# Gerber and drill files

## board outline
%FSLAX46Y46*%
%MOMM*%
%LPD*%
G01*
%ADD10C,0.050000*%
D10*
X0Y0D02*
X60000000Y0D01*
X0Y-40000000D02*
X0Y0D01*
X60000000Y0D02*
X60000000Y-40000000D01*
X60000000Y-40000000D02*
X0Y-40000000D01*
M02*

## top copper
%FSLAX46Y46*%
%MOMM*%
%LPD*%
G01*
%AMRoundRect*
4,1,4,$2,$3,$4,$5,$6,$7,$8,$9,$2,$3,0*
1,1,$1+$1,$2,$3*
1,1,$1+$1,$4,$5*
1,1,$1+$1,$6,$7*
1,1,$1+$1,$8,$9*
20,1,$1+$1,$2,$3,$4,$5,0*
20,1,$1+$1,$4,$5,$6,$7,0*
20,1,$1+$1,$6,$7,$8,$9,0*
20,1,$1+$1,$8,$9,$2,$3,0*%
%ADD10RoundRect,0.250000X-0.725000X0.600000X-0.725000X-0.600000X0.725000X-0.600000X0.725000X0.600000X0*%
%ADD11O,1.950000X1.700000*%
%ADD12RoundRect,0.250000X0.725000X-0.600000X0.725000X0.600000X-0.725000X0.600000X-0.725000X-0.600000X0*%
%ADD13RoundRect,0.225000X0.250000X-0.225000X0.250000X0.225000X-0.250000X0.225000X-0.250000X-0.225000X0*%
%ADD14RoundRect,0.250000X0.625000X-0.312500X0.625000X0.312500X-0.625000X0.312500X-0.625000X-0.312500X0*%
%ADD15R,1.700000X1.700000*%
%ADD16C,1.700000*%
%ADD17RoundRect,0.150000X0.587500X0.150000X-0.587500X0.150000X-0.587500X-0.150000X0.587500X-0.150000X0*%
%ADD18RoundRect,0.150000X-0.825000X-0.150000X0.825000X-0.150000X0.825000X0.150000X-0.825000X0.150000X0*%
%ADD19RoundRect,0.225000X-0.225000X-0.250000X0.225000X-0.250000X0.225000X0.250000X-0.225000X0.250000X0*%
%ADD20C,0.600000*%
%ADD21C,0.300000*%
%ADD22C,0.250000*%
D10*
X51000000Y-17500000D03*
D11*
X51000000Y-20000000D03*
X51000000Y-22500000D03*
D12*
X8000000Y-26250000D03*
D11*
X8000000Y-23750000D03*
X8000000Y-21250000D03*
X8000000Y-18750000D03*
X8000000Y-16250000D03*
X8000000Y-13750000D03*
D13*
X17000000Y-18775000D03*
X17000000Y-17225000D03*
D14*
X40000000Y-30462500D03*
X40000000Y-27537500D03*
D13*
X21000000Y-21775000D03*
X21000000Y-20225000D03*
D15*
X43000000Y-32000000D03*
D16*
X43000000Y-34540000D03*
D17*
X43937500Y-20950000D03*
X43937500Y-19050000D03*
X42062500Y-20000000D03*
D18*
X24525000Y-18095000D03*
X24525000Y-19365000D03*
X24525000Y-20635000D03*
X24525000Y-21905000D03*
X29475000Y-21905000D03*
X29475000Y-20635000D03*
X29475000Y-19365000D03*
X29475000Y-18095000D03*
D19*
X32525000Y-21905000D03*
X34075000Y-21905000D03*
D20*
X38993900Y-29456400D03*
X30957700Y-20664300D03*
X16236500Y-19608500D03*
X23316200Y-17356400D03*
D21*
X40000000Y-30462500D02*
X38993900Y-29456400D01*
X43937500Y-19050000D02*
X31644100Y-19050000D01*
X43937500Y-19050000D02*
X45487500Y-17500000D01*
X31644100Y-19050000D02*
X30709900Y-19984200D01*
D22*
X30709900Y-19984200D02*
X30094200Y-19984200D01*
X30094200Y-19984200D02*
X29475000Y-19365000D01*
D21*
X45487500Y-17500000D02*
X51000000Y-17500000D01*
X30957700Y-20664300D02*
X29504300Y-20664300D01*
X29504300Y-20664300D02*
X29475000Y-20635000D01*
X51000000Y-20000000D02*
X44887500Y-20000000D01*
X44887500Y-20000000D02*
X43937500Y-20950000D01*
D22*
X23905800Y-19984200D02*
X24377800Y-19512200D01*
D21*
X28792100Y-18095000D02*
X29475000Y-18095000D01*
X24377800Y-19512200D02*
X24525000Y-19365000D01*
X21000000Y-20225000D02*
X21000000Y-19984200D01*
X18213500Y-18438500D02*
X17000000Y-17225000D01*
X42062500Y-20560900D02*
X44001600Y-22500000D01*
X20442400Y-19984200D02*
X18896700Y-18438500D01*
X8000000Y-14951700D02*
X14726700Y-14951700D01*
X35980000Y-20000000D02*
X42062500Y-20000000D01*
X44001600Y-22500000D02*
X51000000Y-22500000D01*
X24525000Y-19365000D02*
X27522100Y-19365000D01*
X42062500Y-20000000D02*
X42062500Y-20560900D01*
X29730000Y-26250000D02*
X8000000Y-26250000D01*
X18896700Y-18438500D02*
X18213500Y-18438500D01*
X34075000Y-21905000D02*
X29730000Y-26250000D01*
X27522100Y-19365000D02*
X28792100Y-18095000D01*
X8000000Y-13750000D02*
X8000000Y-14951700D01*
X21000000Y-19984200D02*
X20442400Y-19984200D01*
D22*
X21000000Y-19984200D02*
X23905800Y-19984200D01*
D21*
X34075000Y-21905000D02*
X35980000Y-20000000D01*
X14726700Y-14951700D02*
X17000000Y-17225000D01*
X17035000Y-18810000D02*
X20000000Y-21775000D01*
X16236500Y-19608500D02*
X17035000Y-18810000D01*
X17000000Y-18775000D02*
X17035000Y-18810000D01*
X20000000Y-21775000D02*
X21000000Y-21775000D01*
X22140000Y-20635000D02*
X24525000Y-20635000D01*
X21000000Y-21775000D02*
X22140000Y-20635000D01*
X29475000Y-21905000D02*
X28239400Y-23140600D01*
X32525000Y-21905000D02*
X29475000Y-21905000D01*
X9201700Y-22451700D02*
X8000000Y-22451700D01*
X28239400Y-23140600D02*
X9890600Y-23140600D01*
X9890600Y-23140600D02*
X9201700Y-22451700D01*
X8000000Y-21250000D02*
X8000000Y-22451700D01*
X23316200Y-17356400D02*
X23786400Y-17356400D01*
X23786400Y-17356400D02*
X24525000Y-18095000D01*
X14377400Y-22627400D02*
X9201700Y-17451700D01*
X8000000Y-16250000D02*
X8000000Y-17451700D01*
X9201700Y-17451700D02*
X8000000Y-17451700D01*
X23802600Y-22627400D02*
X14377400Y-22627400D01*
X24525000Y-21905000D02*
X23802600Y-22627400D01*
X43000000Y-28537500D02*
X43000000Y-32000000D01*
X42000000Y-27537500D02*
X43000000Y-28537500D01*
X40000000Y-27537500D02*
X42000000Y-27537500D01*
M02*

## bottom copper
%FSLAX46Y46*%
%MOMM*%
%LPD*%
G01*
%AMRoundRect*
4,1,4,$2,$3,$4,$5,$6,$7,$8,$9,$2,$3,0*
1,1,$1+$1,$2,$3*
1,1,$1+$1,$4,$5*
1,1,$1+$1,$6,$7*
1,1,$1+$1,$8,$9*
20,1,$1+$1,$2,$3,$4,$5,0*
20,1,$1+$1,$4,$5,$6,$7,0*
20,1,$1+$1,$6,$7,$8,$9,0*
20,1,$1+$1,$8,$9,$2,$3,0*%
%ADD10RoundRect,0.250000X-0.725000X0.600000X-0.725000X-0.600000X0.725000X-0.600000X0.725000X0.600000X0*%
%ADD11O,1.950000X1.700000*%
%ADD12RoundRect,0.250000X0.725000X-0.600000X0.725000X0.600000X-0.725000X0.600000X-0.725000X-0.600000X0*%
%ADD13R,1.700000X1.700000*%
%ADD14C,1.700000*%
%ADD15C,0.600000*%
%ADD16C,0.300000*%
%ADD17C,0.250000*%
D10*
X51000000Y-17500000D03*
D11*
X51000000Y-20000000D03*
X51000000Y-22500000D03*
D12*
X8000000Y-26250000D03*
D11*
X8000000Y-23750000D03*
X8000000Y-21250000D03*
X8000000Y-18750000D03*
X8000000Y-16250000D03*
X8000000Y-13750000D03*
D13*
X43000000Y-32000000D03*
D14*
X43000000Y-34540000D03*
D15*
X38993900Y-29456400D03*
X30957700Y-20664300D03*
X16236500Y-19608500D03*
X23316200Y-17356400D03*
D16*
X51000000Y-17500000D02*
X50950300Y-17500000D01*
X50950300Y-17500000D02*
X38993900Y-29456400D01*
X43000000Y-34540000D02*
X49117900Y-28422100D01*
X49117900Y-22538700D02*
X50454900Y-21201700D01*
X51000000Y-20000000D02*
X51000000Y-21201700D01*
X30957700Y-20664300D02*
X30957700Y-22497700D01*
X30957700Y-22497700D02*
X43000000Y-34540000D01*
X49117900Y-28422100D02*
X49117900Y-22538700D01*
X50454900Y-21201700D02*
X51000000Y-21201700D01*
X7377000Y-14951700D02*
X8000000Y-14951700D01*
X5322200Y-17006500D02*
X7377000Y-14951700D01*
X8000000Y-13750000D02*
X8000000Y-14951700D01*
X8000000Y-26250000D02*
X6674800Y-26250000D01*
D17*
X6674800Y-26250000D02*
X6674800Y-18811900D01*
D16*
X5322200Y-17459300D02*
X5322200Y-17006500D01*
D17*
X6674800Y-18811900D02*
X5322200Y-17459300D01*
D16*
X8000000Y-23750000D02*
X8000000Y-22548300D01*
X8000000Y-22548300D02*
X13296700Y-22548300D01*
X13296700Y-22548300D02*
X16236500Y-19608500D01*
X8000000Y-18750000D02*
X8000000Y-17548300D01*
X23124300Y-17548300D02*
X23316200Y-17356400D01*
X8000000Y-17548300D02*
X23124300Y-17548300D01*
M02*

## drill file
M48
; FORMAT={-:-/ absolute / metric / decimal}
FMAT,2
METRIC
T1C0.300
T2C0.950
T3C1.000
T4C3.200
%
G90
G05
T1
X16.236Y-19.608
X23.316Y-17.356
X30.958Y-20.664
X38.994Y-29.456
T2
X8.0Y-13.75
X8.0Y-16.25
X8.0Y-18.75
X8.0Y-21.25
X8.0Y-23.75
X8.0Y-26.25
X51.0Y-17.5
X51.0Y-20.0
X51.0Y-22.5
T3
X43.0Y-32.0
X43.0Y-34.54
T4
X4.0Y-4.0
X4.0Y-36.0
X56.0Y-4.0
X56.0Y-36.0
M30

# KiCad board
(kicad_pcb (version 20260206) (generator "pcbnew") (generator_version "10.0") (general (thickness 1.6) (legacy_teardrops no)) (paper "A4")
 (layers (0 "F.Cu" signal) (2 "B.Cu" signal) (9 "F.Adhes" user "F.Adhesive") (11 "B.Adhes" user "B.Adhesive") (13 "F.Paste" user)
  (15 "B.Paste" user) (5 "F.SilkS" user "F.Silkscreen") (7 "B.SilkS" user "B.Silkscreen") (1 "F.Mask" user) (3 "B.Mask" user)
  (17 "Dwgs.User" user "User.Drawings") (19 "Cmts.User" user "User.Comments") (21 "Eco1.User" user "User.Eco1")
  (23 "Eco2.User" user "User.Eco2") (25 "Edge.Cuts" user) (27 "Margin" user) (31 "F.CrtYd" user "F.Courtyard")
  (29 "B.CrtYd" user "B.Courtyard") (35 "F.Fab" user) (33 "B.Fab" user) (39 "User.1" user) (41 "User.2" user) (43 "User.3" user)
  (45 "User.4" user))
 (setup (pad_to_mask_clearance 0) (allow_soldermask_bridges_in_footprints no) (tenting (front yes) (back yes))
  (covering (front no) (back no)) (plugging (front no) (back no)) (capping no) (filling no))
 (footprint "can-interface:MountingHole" (layer "F.Cu") (at 56 36)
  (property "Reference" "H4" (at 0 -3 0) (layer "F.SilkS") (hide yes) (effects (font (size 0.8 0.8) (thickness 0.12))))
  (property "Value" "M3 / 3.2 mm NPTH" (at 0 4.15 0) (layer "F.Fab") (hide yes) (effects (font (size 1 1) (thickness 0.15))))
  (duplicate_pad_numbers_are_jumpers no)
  (pad "" np_thru_hole circle (at 0 0) (size 3.2 3.2) (drill 3.2) (layers "*.Cu" "*.Mask")))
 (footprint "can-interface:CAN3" (layer "F.Cu") (at 51 17.5 -90)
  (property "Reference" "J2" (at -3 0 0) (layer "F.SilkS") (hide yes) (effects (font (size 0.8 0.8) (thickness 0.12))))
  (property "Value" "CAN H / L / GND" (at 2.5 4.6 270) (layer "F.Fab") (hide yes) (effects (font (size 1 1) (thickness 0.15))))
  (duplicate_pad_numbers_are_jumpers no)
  (pad "1" thru_hole roundrect (at 0 0 270) (size 1.7 1.95) (drill 0.95) (layers "*.Cu" "*.Mask") (remove_unused_layers no)
   (roundrect_rratio 0.147059) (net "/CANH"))
  (pad "2" thru_hole oval (at 2.5 0 270) (size 1.7 1.95) (drill 0.95) (layers "*.Cu" "*.Mask") (remove_unused_layers no) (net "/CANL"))
  (pad "3" thru_hole oval (at 5 0 270) (size 1.7 1.95) (drill 0.95) (layers "*.Cu" "*.Mask") (remove_unused_layers no) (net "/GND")))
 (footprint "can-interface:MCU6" (layer "F.Cu") (at 8 26.25 90)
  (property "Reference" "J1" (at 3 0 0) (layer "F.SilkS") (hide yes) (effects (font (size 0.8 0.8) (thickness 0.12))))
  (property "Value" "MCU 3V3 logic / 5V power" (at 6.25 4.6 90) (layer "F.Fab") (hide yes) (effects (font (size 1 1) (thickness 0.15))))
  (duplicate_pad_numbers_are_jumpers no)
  (pad "1" thru_hole roundrect (at 0 0 90) (size 1.7 1.95) (drill 0.95) (layers "*.Cu" "*.Mask") (remove_unused_layers no)
   (roundrect_rratio 0.147059) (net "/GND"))
  (pad "2" thru_hole oval (at 2.5 0 90) (size 1.7 1.95) (drill 0.95) (layers "*.Cu" "*.Mask") (remove_unused_layers no) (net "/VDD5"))
  (pad "3" thru_hole oval (at 5 0 90) (size 1.7 1.95) (drill 0.95) (layers "*.Cu" "*.Mask") (remove_unused_layers no) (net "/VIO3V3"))
  (pad "4" thru_hole oval (at 7.5 0 90) (size 1.7 1.95) (drill 0.95) (layers "*.Cu" "*.Mask") (remove_unused_layers no) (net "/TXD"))
  (pad "5" thru_hole oval (at 10 0 90) (size 1.7 1.95) (drill 0.95) (layers "*.Cu" "*.Mask") (remove_unused_layers no) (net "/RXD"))
  (pad "6" thru_hole oval (at 12.5 0 90) (size 1.7 1.95) (drill 0.95) (layers "*.Cu" "*.Mask") (remove_unused_layers no) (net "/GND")))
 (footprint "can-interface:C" (layer "F.Cu") (at 17 18 90)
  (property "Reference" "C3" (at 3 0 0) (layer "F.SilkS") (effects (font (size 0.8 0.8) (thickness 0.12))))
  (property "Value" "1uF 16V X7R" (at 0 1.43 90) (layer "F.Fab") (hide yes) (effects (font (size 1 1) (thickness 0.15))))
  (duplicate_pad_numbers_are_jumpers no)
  (pad "1" smd roundrect (at -0.775 0 90) (size 0.9 0.95) (layers "F.Cu" "F.Mask" "F.Paste") (roundrect_rratio 0.25) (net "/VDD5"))
  (pad "2" smd roundrect (at 0.775 0 90) (size 0.9 0.95) (layers "F.Cu" "F.Mask" "F.Paste") (roundrect_rratio 0.25) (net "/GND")))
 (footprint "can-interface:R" (layer "F.Cu") (at 40 29 90)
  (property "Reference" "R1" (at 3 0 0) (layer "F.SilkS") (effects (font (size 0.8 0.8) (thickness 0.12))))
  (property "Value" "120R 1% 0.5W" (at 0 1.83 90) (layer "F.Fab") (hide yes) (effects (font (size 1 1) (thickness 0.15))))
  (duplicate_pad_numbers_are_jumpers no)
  (pad "1" smd roundrect (at -1.4625 0 90) (size 1.125 1.75) (layers "F.Cu" "F.Mask" "F.Paste") (roundrect_rratio 0.222222) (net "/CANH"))
  (pad "2" smd roundrect (at 1.4625 0 90) (size 1.125 1.75) (layers "F.Cu" "F.Mask" "F.Paste") (roundrect_rratio 0.222222) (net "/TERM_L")))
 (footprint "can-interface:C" (layer "F.Cu") (at 21 21 90)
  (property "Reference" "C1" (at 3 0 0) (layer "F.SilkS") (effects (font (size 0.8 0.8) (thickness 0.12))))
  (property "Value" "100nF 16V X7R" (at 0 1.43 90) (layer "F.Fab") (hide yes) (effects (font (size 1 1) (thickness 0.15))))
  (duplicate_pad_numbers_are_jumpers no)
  (pad "1" smd roundrect (at -0.775 0 90) (size 0.9 0.95) (layers "F.Cu" "F.Mask" "F.Paste") (roundrect_rratio 0.25) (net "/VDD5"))
  (pad "2" smd roundrect (at 0.775 0 90) (size 0.9 0.95) (layers "F.Cu" "F.Mask" "F.Paste") (roundrect_rratio 0.25) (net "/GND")))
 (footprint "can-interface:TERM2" (layer "F.Cu") (at 43 32)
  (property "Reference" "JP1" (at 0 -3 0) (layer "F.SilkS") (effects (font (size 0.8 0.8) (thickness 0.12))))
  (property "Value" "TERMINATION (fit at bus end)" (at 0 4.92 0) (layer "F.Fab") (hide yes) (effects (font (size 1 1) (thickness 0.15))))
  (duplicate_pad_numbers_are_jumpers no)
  (pad "1" thru_hole rect (at 0 0) (size 1.7 1.7) (drill 1) (layers "*.Cu" "*.Mask") (remove_unused_layers no) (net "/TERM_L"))
  (pad "2" thru_hole circle (at 0 2.54) (size 1.7 1.7) (drill 1) (layers "*.Cu" "*.Mask") (remove_unused_layers no) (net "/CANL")))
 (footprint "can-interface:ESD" (layer "F.Cu") (at 43 20 180)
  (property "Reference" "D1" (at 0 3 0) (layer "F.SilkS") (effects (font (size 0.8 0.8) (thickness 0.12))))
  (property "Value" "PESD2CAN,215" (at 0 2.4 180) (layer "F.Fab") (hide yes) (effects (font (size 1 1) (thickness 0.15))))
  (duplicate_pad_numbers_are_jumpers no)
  (pad "1" smd roundrect (at -0.9375 -0.95 180) (size 1.475 0.6) (layers "F.Cu" "F.Mask" "F.Paste") (roundrect_rratio 0.25) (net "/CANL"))
  (pad "2" smd roundrect (at -0.9375 0.95 180) (size 1.475 0.6) (layers "F.Cu" "F.Mask" "F.Paste") (roundrect_rratio 0.25) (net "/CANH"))
  (pad "3" smd roundrect (at 0.9375 0 180) (size 1.475 0.6) (layers "F.Cu" "F.Mask" "F.Paste") (roundrect_rratio 0.25) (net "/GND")))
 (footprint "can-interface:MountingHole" (layer "F.Cu") (at 4 36)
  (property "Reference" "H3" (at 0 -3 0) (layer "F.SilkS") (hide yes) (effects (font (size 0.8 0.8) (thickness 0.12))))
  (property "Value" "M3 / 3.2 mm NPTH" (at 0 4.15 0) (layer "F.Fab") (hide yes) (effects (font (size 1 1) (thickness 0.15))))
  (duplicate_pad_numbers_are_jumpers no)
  (pad "" np_thru_hole circle (at 0 0) (size 3.2 3.2) (drill 3.2) (layers "*.Cu" "*.Mask")))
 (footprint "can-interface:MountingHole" (layer "F.Cu") (at 4 4)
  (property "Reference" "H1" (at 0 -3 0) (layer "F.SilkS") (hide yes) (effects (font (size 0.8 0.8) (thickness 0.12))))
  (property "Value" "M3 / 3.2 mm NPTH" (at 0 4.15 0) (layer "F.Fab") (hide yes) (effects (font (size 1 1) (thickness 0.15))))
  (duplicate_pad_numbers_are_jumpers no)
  (pad "" np_thru_hole circle (at 0 0) (size 3.2 3.2) (drill 3.2) (layers "*.Cu" "*.Mask")))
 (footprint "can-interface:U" (layer "F.Cu") (at 27 20)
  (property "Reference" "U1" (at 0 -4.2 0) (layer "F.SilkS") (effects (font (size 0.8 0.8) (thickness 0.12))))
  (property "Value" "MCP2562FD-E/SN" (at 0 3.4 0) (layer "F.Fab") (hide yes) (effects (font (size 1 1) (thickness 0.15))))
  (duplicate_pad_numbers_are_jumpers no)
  (pad "1" smd roundrect (at -2.475 -1.905) (size 1.95 0.6) (layers "F.Cu" "F.Mask" "F.Paste") (roundrect_rratio 0.25) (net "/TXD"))
  (pad "2" smd roundrect (at -2.475 -0.635) (size 1.95 0.6) (layers "F.Cu" "F.Mask" "F.Paste") (roundrect_rratio 0.25) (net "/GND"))
  (pad "3" smd roundrect (at -2.475 0.635) (size 1.95 0.6) (layers "F.Cu" "F.Mask" "F.Paste") (roundrect_rratio 0.25) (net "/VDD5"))
  (pad "4" smd roundrect (at -2.475 1.905) (size 1.95 0.6) (layers "F.Cu" "F.Mask" "F.Paste") (roundrect_rratio 0.25) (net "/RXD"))
  (pad "5" smd roundrect (at 2.475 1.905) (size 1.95 0.6) (layers "F.Cu" "F.Mask" "F.Paste") (roundrect_rratio 0.25) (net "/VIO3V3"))
  (pad "6" smd roundrect (at 2.475 0.635) (size 1.95 0.6) (layers "F.Cu" "F.Mask" "F.Paste") (roundrect_rratio 0.25) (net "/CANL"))
  (pad "7" smd roundrect (at 2.475 -0.635) (size 1.95 0.6) (layers "F.Cu" "F.Mask" "F.Paste") (roundrect_rratio 0.25) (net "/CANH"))
  (pad "8" smd roundrect (at 2.475 -1.905) (size 1.95 0.6) (layers "F.Cu" "F.Mask" "F.Paste") (roundrect_rratio 0.25) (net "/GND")))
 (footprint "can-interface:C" (layer "F.Cu") (at 33.3 21.905)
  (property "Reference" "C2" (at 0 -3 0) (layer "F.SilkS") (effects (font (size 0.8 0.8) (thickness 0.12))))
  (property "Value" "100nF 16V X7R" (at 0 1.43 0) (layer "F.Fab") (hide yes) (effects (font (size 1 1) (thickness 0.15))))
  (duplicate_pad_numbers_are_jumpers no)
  (pad "1" smd roundrect (at -0.775 0) (size 0.9 0.95) (layers "F.Cu" "F.Mask" "F.Paste") (roundrect_rratio 0.25) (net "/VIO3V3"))
  (pad "2" smd roundrect (at 0.775 0) (size 0.9 0.95) (layers "F.Cu" "F.Mask" "F.Paste") (roundrect_rratio 0.25) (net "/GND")))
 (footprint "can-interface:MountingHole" (layer "F.Cu") (at 56 4)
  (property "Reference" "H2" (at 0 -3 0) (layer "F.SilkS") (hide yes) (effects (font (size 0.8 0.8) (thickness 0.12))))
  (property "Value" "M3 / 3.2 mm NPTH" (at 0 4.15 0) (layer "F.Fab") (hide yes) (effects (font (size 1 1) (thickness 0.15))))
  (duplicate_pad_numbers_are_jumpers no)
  (pad "" np_thru_hole circle (at 0 0) (size 3.2 3.2) (drill 3.2) (layers "*.Cu" "*.Mask")))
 (gr_line (start 0 0) (end 60 0) (stroke (width 0.05) (type default)) (layer "Edge.Cuts"))
 (gr_line (start 0 40) (end 0 0) (stroke (width 0.05) (type default)) (layer "Edge.Cuts"))
 (gr_line (start 60 0) (end 60 40) (stroke (width 0.05) (type default)) (layer "Edge.Cuts"))
 (gr_line (start 60 40) (end 0 40) (stroke (width 0.05) (type default)) (layer "Edge.Cuts"))
 (segment (start 40 30.4625) (end 38.9939 29.4564) (width 0.3) (layer "F.Cu") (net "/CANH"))
 (segment (start 43.9375 19.05) (end 31.6441 19.05) (width 0.3) (layer "F.Cu") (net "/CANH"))
 (segment (start 43.9375 19.05) (end 45.4875 17.5) (width 0.3) (layer "F.Cu") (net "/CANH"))
 (segment (start 31.6441 19.05) (end 30.7099 19.9842) (width 0.3) (layer "F.Cu") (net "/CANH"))
 (segment (start 30.7099 19.9842) (end 30.0942 19.9842) (width 0.25) (layer "F.Cu") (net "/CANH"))
 (segment (start 30.0942 19.9842) (end 29.475 19.365) (width 0.25) (layer "F.Cu") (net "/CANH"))
 (segment (start 45.4875 17.5) (end 51 17.5) (width 0.3) (layer "F.Cu") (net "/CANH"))
 (via (at 38.9939 29.4564) (size 0.6) (drill 0.3) (layers "F.Cu" "B.Cu") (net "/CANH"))
 (segment (start 51 17.5) (end 50.9503 17.5) (width 0.3) (layer "B.Cu") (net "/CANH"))
 (segment (start 50.9503 17.5) (end 38.9939 29.4564) (width 0.3) (layer "B.Cu") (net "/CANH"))
 (segment (start 30.9577 20.6643) (end 29.5043 20.6643) (width 0.3) (layer "F.Cu") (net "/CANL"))
 (segment (start 29.5043 20.6643) (end 29.475 20.635) (width 0.3) (layer "F.Cu") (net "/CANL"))
 (segment (start 51 20) (end 44.8875 20) (width 0.3) (layer "F.Cu") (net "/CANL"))
 (segment (start 44.8875 20) (end 43.9375 20.95) (width 0.3) (layer "F.Cu") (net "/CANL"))
 (via (at 30.9577 20.6643) (size 0.6) (drill 0.3) (layers "F.Cu" "B.Cu") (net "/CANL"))
 (segment (start 43 34.54) (end 49.1179 28.4221) (width 0.3) (layer "B.Cu") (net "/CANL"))
 (segment (start 49.1179 22.5387) (end 50.4549 21.2017) (width 0.3) (layer "B.Cu") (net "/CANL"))
 (segment (start 51 20) (end 51 21.2017) (width 0.3) (layer "B.Cu") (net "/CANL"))
 (segment (start 30.9577 20.6643) (end 30.9577 22.4977) (width 0.3) (layer "B.Cu") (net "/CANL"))
 (segment (start 30.9577 22.4977) (end 43 34.54) (width 0.3) (layer "B.Cu") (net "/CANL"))
 (segment (start 49.1179 28.4221) (end 49.1179 22.5387) (width 0.3) (layer "B.Cu") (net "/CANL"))
 (segment (start 50.4549 21.2017) (end 51 21.2017) (width 0.3) (layer "B.Cu") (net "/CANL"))
 (segment (start 23.9058 19.9842) (end 24.3778 19.5122) (width 0.25) (layer "F.Cu") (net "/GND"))
 (segment (start 28.7921 18.095) (end 29.475 18.095) (width 0.3) (layer "F.Cu") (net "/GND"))
 (segment (start 24.3778 19.5122) (end 24.525 19.365) (width 0.3) (layer "F.Cu") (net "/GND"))
 (segment (start 21 20.225) (end 21 19.9842) (width 0.3) (layer "F.Cu") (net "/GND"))
 (segment (start 18.2135 18.4385) (end 17 17.225) (width 0.3) (layer "F.Cu") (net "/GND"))
 (segment (start 42.0625 20.5609) (end 44.0016 22.5) (width 0.3) (layer "F.Cu") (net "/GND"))
 (segment (start 20.4424 19.9842) (end 18.8967 18.4385) (width 0.3) (layer "F.Cu") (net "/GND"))
 (segment (start 8 14.9517) (end 14.7267 14.9517) (width 0.3) (layer "F.Cu") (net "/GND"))
 (segment (start 35.98 20) (end 42.0625 20) (width 0.3) (layer "F.Cu") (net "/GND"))
 (segment (start 44.0016 22.5) (end 51 22.5) (width 0.3) (layer "F.Cu") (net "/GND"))
 (segment (start 24.525 19.365) (end 27.5221 19.365) (width 0.3) (layer "F.Cu") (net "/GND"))
 (segment (start 42.0625 20) (end 42.0625 20.5609) (width 0.3) (layer "F.Cu") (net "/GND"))
 (segment (start 29.73 26.25) (end 8 26.25) (width 0.3) (layer "F.Cu") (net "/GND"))
 (segment (start 18.8967 18.4385) (end 18.2135 18.4385) (width 0.3) (layer "F.Cu") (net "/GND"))
 (segment (start 34.075 21.905) (end 29.73 26.25) (width 0.3) (layer "F.Cu") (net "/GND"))
 (segment (start 27.5221 19.365) (end 28.7921 18.095) (width 0.3) (layer "F.Cu") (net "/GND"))
 (segment (start 8 13.75) (end 8 14.9517) (width 0.3) (layer "F.Cu") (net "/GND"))
 (segment (start 21 19.9842) (end 20.4424 19.9842) (width 0.3) (layer "F.Cu") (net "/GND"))
 (segment (start 21 19.9842) (end 23.9058 19.9842) (width 0.25) (layer "F.Cu") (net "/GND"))
 (segment (start 34.075 21.905) (end 35.98 20) (width 0.3) (layer "F.Cu") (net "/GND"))
 (segment (start 14.7267 14.9517) (end 17 17.225) (width 0.3) (layer "F.Cu") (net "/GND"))
 (segment (start 7.377 14.9517) (end 8 14.9517) (width 0.3) (layer "B.Cu") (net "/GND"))
 (segment (start 5.3222 17.0065) (end 7.377 14.9517) (width 0.3) (layer "B.Cu") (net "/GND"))
 (segment (start 8 13.75) (end 8 14.9517) (width 0.3) (layer "B.Cu") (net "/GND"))
 (segment (start 8 26.25) (end 6.6748 26.25) (width 0.3) (layer "B.Cu") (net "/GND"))
 (segment (start 6.6748 26.25) (end 6.6748 18.8119) (width 0.25) (layer "B.Cu") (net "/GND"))
 (segment (start 5.3222 17.4593) (end 5.3222 17.0065) (width 0.3) (layer "B.Cu") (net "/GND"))
 (segment (start 6.6748 18.8119) (end 5.3222 17.4593) (width 0.25) (layer "B.Cu") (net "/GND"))
 (segment (start 17.035 18.81) (end 20 21.775) (width 0.3) (layer "F.Cu") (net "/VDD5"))
 (segment (start 16.2365 19.6085) (end 17.035 18.81) (width 0.3) (layer "F.Cu") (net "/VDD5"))
 (segment (start 17 18.775) (end 17.035 18.81) (width 0.3) (layer "F.Cu") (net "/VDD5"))
 (segment (start 20 21.775) (end 21 21.775) (width 0.3) (layer "F.Cu") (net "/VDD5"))
 (segment (start 22.14 20.635) (end 24.525 20.635) (width 0.3) (layer "F.Cu") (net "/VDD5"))
 (segment (start 21 21.775) (end 22.14 20.635) (width 0.3) (layer "F.Cu") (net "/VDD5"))
 (via (at 16.2365 19.6085) (size 0.6) (drill 0.3) (layers "F.Cu" "B.Cu") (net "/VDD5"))
 (segment (start 8 23.75) (end 8 22.5483) (width 0.3) (layer "B.Cu") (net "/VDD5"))
 (segment (start 8 22.5483) (end 13.2967 22.5483) (width 0.3) (layer "B.Cu") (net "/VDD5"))
 (segment (start 13.2967 22.5483) (end 16.2365 19.6085) (width 0.3) (layer "B.Cu") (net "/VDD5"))
 (segment (start 29.475 21.905) (end 28.2394 23.1406) (width 0.3) (layer "F.Cu") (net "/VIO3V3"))
 (segment (start 32.525 21.905) (end 29.475 21.905) (width 0.3) (layer "F.Cu") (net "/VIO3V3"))
 (segment (start 9.2017 22.4517) (end 8 22.4517) (width 0.3) (layer "F.Cu") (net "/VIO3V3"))
 (segment (start 28.2394 23.1406) (end 9.8906 23.1406) (width 0.3) (layer "F.Cu") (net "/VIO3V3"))
 (segment (start 9.8906 23.1406) (end 9.2017 22.4517) (width 0.3) (layer "F.Cu") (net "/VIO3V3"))
 (segment (start 8 21.25) (end 8 22.4517) (width 0.3) (layer "F.Cu") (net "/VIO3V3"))
 (segment (start 23.3162 17.3564) (end 23.7864 17.3564) (width 0.3) (layer "F.Cu") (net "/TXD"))
 (segment (start 23.7864 17.3564) (end 24.525 18.095) (width 0.3) (layer "F.Cu") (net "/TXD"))
 (via (at 23.3162 17.3564) (size 0.6) (drill 0.3) (layers "F.Cu" "B.Cu") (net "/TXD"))
 (segment (start 8 18.75) (end 8 17.5483) (width 0.3) (layer "B.Cu") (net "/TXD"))
 (segment (start 23.1243 17.5483) (end 23.3162 17.3564) (width 0.3) (layer "B.Cu") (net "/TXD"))
 (segment (start 8 17.5483) (end 23.1243 17.5483) (width 0.3) (layer "B.Cu") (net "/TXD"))
 (segment (start 14.3774 22.6274) (end 9.2017 17.4517) (width 0.3) (layer "F.Cu") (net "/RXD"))
 (segment (start 8 16.25) (end 8 17.4517) (width 0.3) (layer "F.Cu") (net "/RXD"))
 (segment (start 9.2017 17.4517) (end 8 17.4517) (width 0.3) (layer "F.Cu") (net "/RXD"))
 (segment (start 23.8026 22.6274) (end 14.3774 22.6274) (width 0.3) (layer "F.Cu") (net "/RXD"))
 (segment (start 24.525 21.905) (end 23.8026 22.6274) (width 0.3) (layer "F.Cu") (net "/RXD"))
 (segment (start 43 28.5375) (end 43 32) (width 0.3) (layer "F.Cu") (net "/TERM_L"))
 (segment (start 42 27.5375) (end 43 28.5375) (width 0.3) (layer "F.Cu") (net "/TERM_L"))
 (segment (start 40 27.5375) (end 42 27.5375) (width 0.3) (layer "F.Cu") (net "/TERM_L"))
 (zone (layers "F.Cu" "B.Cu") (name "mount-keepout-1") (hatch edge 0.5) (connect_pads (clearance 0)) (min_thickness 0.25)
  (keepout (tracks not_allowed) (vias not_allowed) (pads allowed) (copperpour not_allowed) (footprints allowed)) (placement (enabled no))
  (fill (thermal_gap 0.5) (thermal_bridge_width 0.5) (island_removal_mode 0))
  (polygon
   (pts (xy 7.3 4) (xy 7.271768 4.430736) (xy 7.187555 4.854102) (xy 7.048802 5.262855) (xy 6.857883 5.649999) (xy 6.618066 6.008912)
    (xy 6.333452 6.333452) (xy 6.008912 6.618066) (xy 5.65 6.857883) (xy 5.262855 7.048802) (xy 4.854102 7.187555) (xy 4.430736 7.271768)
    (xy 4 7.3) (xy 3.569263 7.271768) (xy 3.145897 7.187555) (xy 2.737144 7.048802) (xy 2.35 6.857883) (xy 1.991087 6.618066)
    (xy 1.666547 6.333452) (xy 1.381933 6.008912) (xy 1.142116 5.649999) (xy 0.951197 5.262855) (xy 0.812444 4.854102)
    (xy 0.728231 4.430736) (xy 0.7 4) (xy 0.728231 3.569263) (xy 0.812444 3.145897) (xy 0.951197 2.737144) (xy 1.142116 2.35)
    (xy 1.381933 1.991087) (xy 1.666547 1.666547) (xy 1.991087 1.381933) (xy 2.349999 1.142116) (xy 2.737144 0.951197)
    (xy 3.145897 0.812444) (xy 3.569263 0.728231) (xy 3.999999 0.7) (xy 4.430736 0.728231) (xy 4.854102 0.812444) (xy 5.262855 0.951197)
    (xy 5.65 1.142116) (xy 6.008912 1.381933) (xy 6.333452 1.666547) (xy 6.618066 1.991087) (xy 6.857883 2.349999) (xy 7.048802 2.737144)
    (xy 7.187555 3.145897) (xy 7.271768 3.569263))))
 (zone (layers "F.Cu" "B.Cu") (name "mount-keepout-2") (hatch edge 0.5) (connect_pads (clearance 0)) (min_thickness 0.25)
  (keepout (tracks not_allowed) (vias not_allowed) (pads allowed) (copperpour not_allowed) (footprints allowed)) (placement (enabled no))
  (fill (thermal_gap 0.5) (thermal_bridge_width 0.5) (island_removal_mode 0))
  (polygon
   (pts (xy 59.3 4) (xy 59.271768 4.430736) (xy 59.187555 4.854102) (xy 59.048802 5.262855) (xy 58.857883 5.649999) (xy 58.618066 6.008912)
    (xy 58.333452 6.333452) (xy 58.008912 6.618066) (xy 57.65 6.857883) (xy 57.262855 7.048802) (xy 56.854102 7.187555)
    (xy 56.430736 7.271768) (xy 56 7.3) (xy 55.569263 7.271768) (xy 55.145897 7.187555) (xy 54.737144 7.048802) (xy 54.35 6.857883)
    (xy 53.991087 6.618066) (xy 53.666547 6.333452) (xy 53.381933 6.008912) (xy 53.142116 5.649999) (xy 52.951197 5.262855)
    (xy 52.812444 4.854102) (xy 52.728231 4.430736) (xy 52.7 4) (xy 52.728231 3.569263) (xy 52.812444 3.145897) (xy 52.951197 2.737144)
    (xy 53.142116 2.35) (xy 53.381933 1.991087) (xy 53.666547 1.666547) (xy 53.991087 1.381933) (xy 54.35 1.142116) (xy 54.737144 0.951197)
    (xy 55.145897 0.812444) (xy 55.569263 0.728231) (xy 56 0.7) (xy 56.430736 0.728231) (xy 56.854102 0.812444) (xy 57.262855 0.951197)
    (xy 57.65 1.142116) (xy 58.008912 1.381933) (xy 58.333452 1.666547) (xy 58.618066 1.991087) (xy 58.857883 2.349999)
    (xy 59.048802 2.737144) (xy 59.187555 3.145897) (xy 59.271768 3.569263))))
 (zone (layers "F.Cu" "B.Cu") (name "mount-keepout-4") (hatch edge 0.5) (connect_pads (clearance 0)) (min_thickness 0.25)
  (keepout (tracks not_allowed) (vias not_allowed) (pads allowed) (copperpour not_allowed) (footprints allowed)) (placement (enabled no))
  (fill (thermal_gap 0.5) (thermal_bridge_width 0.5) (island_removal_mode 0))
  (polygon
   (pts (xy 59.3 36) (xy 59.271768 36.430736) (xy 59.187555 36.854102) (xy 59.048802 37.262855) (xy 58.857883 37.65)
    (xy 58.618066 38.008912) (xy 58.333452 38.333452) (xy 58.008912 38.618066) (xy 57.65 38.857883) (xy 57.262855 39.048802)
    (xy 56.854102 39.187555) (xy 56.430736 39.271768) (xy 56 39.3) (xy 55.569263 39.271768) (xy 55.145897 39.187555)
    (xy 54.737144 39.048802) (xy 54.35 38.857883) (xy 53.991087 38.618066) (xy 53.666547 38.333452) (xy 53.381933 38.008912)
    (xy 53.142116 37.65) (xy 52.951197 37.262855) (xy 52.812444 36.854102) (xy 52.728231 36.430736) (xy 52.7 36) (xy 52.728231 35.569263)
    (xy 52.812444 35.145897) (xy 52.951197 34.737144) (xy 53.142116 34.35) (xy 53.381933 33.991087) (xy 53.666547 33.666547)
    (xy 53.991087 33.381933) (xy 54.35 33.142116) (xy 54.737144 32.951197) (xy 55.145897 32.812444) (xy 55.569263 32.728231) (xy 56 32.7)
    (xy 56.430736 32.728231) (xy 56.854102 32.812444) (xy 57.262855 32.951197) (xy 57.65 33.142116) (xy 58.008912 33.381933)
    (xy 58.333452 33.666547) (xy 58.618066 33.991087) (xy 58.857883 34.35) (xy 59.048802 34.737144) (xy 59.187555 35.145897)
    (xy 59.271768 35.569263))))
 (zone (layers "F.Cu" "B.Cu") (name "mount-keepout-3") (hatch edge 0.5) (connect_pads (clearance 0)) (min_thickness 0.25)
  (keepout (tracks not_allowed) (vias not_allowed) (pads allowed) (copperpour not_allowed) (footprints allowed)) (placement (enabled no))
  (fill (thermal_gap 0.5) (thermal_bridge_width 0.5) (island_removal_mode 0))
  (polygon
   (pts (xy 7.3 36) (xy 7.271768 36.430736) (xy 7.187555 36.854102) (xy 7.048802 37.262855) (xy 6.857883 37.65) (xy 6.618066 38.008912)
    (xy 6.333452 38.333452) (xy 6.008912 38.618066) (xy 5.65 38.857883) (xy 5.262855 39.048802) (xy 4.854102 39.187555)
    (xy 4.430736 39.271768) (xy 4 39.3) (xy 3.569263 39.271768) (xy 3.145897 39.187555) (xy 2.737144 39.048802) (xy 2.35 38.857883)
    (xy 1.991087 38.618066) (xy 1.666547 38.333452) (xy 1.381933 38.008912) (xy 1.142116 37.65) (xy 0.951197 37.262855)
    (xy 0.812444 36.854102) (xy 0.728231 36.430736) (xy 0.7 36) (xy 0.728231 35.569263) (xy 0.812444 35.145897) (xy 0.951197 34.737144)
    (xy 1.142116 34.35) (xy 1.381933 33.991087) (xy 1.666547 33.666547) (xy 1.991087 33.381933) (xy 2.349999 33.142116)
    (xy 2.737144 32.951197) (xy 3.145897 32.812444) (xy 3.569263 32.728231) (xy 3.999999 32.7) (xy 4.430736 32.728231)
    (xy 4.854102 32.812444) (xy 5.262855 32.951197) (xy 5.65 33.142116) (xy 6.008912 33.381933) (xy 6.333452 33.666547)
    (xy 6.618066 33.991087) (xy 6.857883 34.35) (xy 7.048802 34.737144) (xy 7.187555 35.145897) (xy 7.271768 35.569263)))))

